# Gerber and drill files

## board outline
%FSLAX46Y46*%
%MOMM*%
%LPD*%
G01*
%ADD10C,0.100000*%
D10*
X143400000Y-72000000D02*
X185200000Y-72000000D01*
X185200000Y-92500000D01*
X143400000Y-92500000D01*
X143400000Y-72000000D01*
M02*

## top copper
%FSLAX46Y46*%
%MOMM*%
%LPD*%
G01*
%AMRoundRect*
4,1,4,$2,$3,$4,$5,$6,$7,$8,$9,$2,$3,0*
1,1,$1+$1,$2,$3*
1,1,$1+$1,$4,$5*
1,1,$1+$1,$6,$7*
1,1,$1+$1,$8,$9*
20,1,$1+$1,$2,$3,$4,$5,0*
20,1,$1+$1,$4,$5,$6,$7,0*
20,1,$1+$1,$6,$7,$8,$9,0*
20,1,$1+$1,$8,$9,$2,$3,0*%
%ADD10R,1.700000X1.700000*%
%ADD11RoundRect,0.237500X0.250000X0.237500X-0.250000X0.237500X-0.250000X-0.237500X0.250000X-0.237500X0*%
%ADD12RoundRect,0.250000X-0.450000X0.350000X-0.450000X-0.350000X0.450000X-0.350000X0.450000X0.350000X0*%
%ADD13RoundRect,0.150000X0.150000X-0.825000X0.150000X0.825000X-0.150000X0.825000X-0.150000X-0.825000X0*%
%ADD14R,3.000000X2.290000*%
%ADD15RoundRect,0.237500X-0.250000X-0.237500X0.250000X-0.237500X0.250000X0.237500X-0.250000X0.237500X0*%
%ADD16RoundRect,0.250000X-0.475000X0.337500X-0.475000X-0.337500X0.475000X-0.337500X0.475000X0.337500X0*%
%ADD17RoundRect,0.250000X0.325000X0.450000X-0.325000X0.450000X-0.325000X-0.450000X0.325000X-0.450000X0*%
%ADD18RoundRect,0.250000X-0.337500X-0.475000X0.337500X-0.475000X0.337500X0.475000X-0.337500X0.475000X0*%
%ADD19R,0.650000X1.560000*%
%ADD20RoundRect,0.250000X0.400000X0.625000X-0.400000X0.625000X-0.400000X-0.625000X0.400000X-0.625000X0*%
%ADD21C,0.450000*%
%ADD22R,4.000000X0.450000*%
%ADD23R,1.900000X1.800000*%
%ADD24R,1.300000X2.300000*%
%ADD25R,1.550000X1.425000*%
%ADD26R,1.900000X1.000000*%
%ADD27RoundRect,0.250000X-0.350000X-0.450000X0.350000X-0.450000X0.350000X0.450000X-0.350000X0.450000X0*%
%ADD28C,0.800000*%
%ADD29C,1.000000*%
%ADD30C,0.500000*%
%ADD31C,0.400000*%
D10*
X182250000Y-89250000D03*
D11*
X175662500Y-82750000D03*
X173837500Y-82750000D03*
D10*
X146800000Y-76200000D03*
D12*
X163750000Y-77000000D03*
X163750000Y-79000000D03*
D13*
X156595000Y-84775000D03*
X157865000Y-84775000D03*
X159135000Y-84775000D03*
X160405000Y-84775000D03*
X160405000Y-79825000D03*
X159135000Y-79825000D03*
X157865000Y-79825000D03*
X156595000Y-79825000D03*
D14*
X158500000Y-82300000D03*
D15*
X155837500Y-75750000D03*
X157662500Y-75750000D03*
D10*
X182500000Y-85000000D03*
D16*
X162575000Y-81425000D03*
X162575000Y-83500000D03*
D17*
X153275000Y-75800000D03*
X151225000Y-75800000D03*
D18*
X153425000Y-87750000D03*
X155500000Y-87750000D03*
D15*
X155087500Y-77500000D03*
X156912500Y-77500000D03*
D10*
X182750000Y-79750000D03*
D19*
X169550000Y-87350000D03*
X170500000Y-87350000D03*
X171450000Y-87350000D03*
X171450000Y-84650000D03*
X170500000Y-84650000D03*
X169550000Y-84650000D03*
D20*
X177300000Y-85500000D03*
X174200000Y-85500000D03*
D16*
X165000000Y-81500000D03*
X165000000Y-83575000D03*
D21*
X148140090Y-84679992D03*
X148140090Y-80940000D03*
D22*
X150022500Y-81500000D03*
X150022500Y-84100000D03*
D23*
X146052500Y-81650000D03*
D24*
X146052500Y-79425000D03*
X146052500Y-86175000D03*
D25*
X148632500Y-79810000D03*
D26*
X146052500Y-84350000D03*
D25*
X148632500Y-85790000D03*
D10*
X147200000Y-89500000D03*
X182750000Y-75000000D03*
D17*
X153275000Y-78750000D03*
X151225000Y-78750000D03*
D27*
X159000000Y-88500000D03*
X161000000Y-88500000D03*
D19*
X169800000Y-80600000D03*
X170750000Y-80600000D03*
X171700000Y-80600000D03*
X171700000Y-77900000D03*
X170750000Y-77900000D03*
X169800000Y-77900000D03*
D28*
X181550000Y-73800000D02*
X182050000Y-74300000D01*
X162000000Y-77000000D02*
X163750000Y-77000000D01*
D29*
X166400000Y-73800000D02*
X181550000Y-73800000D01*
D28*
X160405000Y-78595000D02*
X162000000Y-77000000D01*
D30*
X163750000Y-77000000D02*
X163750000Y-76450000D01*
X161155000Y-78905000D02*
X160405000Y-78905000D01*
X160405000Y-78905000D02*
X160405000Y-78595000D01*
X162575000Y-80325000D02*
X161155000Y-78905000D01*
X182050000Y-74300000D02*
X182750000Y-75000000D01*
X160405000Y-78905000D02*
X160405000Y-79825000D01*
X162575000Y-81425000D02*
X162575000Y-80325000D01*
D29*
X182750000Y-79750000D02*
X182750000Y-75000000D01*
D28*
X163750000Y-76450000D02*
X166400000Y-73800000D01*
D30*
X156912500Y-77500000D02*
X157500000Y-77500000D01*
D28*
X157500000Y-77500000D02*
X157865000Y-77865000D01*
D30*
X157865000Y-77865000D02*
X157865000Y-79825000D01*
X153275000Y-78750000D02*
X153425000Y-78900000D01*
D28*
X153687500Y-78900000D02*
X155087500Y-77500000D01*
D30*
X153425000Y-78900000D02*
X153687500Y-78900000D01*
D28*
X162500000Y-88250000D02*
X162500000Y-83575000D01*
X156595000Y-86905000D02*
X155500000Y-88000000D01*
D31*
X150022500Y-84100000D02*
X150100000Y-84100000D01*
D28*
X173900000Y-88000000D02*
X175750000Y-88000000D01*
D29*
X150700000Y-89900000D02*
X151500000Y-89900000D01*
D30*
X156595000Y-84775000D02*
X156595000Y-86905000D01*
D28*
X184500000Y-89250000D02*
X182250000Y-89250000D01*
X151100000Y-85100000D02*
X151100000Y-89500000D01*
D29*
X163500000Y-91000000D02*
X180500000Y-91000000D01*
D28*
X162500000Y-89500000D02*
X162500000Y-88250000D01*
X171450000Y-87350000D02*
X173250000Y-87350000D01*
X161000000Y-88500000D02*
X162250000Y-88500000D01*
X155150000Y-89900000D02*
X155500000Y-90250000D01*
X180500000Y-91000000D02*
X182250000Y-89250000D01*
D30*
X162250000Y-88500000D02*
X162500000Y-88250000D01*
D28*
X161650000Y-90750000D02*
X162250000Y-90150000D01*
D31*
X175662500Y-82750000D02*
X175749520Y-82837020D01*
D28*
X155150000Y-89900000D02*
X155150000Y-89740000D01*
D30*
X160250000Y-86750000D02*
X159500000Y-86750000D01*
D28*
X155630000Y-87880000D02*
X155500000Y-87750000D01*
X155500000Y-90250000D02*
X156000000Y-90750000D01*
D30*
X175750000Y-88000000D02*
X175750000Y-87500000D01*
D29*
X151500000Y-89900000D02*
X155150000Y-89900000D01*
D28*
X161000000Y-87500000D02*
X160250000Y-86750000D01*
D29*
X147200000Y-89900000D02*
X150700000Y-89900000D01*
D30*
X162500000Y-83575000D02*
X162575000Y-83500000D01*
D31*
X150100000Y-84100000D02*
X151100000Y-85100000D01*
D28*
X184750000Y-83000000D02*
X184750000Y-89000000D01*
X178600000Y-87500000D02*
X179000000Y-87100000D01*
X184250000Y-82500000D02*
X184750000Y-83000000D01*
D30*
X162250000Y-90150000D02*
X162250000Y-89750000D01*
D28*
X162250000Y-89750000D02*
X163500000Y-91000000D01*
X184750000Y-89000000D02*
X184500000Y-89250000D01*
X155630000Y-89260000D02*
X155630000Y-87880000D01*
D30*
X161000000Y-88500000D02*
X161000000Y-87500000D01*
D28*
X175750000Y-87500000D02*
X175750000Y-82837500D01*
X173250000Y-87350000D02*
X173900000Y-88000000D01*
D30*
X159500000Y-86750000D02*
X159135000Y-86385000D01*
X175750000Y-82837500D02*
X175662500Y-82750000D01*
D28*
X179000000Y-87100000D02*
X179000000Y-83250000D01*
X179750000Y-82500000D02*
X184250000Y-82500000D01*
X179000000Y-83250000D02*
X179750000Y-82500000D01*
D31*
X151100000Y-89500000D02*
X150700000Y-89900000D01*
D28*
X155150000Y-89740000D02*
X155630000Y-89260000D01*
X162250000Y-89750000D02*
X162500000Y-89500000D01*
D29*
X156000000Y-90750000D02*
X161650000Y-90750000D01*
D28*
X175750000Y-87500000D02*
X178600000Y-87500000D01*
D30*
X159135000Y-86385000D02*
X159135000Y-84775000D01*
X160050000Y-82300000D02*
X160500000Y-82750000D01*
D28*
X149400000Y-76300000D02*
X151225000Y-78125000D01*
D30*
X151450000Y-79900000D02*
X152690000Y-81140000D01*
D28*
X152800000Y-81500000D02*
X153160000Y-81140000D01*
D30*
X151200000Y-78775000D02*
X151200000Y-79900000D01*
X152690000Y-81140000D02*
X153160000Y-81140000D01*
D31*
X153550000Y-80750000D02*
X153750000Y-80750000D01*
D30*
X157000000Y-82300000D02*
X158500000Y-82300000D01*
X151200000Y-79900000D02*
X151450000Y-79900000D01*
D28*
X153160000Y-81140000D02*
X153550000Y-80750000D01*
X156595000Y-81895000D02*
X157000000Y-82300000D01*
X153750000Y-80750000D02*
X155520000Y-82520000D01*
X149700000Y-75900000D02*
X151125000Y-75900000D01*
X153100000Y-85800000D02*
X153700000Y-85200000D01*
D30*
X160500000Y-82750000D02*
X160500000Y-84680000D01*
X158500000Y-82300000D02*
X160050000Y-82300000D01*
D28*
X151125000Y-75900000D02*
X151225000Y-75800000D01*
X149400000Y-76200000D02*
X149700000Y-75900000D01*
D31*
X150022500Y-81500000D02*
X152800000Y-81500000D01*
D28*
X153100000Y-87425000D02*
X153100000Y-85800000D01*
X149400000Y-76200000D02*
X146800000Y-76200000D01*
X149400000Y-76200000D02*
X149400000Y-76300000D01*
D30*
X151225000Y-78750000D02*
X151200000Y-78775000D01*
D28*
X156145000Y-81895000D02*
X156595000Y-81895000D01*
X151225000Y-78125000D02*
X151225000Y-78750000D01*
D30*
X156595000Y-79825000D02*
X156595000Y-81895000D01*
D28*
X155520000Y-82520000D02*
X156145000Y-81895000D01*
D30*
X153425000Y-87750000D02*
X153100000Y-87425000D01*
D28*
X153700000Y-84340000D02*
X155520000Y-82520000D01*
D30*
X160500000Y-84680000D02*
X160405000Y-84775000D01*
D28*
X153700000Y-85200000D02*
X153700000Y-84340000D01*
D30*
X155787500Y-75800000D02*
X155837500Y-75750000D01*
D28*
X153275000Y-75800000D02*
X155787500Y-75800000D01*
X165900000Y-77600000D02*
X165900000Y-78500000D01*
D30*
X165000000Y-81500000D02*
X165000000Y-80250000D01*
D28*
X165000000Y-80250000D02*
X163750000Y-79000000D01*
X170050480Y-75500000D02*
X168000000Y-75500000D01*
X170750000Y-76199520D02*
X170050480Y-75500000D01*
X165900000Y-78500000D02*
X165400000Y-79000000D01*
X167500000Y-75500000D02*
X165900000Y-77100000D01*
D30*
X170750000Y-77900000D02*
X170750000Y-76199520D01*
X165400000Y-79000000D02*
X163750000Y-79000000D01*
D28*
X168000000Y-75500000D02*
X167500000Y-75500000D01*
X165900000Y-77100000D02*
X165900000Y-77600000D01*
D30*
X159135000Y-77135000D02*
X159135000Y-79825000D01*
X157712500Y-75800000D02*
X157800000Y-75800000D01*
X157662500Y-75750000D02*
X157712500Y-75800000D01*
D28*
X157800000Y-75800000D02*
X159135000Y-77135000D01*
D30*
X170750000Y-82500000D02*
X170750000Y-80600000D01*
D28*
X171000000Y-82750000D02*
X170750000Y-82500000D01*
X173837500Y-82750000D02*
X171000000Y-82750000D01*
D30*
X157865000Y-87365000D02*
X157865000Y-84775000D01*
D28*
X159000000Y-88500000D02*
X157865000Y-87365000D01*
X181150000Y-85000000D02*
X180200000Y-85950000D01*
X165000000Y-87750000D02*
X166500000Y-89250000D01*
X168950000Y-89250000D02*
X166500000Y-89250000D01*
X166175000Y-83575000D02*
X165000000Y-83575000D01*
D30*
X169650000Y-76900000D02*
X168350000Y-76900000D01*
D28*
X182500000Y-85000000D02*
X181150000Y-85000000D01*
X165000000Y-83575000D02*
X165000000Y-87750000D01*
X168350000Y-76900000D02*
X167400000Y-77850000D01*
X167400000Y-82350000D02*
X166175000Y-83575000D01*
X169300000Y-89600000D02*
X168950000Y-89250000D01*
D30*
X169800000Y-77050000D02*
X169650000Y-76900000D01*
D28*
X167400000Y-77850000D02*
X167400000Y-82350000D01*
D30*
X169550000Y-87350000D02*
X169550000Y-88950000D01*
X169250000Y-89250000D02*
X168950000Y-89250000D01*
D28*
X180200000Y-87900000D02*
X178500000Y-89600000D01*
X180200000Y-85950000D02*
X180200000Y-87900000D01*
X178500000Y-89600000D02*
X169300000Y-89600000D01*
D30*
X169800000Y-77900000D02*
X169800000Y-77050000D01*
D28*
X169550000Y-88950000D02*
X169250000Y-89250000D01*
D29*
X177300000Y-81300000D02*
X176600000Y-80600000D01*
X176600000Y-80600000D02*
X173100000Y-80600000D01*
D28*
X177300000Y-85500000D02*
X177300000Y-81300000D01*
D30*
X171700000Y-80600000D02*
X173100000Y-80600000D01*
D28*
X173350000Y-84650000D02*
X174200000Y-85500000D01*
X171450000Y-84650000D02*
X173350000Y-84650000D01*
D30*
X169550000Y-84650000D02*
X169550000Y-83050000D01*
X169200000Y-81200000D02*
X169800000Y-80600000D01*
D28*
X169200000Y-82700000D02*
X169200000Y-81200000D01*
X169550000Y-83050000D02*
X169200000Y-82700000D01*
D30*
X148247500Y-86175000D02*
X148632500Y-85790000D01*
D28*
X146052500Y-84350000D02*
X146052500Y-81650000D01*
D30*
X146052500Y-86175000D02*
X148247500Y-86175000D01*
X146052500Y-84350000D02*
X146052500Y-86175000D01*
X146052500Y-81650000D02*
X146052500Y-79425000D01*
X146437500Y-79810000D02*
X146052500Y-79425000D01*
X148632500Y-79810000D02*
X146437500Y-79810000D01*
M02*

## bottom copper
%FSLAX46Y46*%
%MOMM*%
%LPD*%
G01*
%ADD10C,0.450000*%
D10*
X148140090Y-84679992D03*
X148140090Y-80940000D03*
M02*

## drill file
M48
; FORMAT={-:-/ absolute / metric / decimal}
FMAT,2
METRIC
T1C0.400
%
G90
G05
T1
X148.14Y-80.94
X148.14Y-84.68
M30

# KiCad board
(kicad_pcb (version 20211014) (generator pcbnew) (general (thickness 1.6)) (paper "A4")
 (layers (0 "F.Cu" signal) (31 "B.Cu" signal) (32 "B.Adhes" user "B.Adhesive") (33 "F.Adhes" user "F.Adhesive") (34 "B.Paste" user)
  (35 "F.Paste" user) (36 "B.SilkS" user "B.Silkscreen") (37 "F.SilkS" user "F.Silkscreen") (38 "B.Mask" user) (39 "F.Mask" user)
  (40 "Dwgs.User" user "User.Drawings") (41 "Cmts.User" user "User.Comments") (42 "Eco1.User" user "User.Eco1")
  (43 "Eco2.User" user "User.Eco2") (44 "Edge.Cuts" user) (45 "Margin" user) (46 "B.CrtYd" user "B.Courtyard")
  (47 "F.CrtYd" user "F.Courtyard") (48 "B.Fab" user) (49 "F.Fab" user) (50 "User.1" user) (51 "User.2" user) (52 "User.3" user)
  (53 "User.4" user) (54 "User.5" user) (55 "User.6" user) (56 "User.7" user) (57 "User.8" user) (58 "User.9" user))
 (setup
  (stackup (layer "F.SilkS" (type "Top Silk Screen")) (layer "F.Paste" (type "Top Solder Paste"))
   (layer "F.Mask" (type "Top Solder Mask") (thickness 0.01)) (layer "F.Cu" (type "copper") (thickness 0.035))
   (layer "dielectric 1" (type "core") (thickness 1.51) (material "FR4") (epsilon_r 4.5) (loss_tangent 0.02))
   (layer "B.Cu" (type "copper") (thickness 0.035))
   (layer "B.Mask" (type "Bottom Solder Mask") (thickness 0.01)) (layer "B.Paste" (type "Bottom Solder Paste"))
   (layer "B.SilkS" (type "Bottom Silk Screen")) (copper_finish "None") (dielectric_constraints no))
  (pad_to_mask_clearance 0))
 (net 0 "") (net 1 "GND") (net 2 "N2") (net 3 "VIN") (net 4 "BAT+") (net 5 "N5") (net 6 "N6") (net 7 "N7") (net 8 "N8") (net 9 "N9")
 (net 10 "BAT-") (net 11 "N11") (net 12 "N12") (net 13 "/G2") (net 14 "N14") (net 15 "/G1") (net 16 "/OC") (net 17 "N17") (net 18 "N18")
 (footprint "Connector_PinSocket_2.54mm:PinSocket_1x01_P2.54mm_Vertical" (layer "F.Cu") (at 182.25 89.25)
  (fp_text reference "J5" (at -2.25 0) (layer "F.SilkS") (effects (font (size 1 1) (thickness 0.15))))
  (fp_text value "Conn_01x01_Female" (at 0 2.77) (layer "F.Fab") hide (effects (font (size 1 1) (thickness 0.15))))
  (pad "1" smd rect (at 0 0) (size 1.7 1.7) (layers "F.Cu" "F.Paste" "F.Mask") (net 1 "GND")))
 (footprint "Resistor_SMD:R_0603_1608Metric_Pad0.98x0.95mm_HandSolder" (layer "F.Cu") (at 174.75 82.75 180)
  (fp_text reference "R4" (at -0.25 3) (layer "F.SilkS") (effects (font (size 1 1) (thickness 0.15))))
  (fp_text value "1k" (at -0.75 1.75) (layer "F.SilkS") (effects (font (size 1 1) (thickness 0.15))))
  (pad "1" smd roundrect (at -0.9125 0 180) (size 0.975 0.95) (layers "F.Cu" "F.Paste" "F.Mask") (roundrect_rratio 0.25) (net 1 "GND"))
  (pad "2" smd roundrect (at 0.9125 0 180) (size 0.975 0.95) (layers "F.Cu" "F.Paste" "F.Mask") (roundrect_rratio 0.25) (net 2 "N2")))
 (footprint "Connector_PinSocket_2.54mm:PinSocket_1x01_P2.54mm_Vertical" (layer "F.Cu") (at 146.8 76.2)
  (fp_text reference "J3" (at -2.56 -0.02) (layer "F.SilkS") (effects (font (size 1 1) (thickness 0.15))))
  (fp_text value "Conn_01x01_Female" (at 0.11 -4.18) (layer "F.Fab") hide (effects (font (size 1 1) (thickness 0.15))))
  (pad "1" smd rect (at 0 0) (size 1.7 1.7) (layers "F.Cu" "F.Paste" "F.Mask") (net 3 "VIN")))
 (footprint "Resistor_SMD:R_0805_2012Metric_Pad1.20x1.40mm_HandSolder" (layer "F.Cu") (at 163.75 78 -90)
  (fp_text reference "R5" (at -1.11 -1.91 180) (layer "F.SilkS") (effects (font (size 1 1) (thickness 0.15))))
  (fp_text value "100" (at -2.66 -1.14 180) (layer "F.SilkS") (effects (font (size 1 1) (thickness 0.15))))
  (pad "1" smd roundrect (at -1 0 270) (size 1.2 1.4) (layers "F.Cu" "F.Paste" "F.Mask") (roundrect_rratio 0.2083333333) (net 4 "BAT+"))
  (pad "2" smd roundrect (at 1 0 270) (size 1.2 1.4) (layers "F.Cu" "F.Paste" "F.Mask") (roundrect_rratio 0.2083333333) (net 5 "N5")))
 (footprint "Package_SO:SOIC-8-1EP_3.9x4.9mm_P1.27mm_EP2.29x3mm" (layer "F.Cu") (at 158.5 82.3 90)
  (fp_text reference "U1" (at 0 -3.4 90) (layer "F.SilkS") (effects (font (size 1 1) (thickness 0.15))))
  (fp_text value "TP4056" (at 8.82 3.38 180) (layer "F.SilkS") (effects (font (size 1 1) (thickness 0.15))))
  (pad "" smd roundrect (at 0.57 0.75 90) (size 0.92 1.21) (layers "F.Paste") (roundrect_rratio 0.25))
  (pad "" smd roundrect (at 0.57 -0.75 90) (size 0.92 1.21) (layers "F.Paste") (roundrect_rratio 0.25))
  (pad "" smd roundrect (at -0.57 0.75 90) (size 0.92 1.21) (layers "F.Paste") (roundrect_rratio 0.25))
  (pad "" smd roundrect (at -0.57 -0.75 90) (size 0.92 1.21) (layers "F.Paste") (roundrect_rratio 0.25))
  (pad "1" smd roundrect (at -2.475 -1.905 90) (size 1.95 0.6) (layers "F.Cu" "F.Paste" "F.Mask") (roundrect_rratio 0.25) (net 1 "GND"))
  (pad "2" smd roundrect (at -2.475 -0.635 90) (size 1.95 0.6) (layers "F.Cu" "F.Paste" "F.Mask") (roundrect_rratio 0.25) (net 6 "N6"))
  (pad "3" smd roundrect (at -2.475 0.635 90) (size 1.95 0.6) (layers "F.Cu" "F.Paste" "F.Mask") (roundrect_rratio 0.25) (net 1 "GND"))
  (pad "4" smd roundrect (at -2.475 1.905 90) (size 1.95 0.6) (layers "F.Cu" "F.Paste" "F.Mask") (roundrect_rratio 0.25) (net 3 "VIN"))
  (pad "5" smd roundrect (at 2.475 1.905 90) (size 1.95 0.6) (layers "F.Cu" "F.Paste" "F.Mask") (roundrect_rratio 0.25) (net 4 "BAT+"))
  (pad "6" smd roundrect (at 2.475 0.635 90) (size 1.95 0.6) (layers "F.Cu" "F.Paste" "F.Mask") (roundrect_rratio 0.25) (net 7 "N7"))
  (pad "7" smd roundrect (at 2.475 -0.635 90) (size 1.95 0.6) (layers "F.Cu" "F.Paste" "F.Mask") (roundrect_rratio 0.25) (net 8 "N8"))
  (pad "8" smd roundrect (at 2.475 -1.905 90) (size 1.95 0.6) (layers "F.Cu" "F.Paste" "F.Mask") (roundrect_rratio 0.25) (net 3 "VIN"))
  (pad "9" smd rect (at 0 0 90) (size 2.29 3) (layers "F.Cu" "F.Mask") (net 3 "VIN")))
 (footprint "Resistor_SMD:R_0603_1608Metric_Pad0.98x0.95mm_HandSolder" (layer "F.Cu") (at 156.75 75.75)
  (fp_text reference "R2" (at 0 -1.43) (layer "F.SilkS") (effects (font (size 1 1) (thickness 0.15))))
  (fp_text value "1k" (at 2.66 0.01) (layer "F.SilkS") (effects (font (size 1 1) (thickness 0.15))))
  (pad "1" smd roundrect (at -0.9125 0) (size 0.975 0.95) (layers "F.Cu" "F.Paste" "F.Mask") (roundrect_rratio 0.25) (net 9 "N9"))
  (pad "2" smd roundrect (at 0.9125 0) (size 0.975 0.95) (layers "F.Cu" "F.Paste" "F.Mask") (roundrect_rratio 0.25) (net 7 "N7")))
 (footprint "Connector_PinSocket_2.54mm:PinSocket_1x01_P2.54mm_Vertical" (layer "F.Cu") (at 182.5 85)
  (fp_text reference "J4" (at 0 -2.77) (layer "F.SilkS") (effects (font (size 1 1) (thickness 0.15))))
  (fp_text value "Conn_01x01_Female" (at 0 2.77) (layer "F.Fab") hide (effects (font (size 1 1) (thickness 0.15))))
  (pad "1" smd rect (at 0 0) (size 1.7 1.7) (layers "F.Cu" "F.Paste" "F.Mask") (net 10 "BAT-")))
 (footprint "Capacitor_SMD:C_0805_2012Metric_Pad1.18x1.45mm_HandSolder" (layer "F.Cu") (at 162.575 82.4625 -90)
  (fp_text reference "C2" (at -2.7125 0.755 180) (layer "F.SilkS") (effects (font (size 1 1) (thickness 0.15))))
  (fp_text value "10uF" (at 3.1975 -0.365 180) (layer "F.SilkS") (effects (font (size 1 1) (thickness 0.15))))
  (pad "1" smd roundrect (at -1.0375 0 270) (size 1.175 1.45) (layers "F.Cu" "F.Paste" "F.Mask") (roundrect_rratio 0.2127659574)
   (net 4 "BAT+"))
  (pad "2" smd roundrect (at 1.0375 0 270) (size 1.175 1.45) (layers "F.Cu" "F.Paste" "F.Mask") (roundrect_rratio 0.2127659574)
   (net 1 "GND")))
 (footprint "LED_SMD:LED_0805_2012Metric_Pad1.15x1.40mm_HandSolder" (layer "F.Cu") (at 152.25 75.8 180)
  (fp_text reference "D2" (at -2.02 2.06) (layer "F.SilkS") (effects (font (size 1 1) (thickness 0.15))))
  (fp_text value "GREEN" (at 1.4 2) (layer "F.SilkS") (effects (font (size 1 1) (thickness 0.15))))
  (pad "1" smd roundrect (at -1.025 0 180) (size 1.15 1.4) (layers "F.Cu" "F.Paste" "F.Mask") (roundrect_rratio 0.2173913043) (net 9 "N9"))
  (pad "2" smd roundrect (at 1.025 0 180) (size 1.15 1.4) (layers "F.Cu" "F.Paste" "F.Mask") (roundrect_rratio 0.2173913043) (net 3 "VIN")))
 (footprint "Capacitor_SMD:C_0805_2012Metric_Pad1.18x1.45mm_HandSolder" (layer "F.Cu") (at 154.4625 87.75)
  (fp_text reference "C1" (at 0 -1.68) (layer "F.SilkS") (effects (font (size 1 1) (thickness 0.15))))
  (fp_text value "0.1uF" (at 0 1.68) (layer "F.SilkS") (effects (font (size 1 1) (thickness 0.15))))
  (pad "1" smd roundrect (at -1.0375 0) (size 1.175 1.45) (layers "F.Cu" "F.Paste" "F.Mask") (roundrect_rratio 0.2127659574) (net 3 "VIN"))
  (pad "2" smd roundrect (at 1.0375 0) (size 1.175 1.45) (layers "F.Cu" "F.Paste" "F.Mask") (roundrect_rratio 0.2127659574) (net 1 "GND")))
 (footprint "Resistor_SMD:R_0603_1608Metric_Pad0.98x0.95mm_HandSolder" (layer "F.Cu") (at 156 77.5)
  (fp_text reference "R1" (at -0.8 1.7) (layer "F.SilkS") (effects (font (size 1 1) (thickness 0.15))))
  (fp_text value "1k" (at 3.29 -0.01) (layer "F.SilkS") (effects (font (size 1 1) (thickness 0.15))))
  (pad "1" smd roundrect (at -0.9125 0) (size 0.975 0.95) (layers "F.Cu" "F.Paste" "F.Mask") (roundrect_rratio 0.25) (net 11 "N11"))
  (pad "2" smd roundrect (at 0.9125 0) (size 0.975 0.95) (layers "F.Cu" "F.Paste" "F.Mask") (roundrect_rratio 0.25) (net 8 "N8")))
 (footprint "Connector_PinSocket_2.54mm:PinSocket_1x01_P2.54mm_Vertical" (layer "F.Cu") (at 182.75 79.75)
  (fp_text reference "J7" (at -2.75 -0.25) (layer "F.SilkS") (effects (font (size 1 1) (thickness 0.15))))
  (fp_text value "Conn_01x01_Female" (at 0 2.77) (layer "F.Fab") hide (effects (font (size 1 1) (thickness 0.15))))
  (pad "1" smd rect (at 0 0) (size 1.7 1.7) (layers "F.Cu" "F.Paste" "F.Mask") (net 4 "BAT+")))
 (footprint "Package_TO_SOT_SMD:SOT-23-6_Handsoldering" (layer "F.Cu") (at 170.5 86 90)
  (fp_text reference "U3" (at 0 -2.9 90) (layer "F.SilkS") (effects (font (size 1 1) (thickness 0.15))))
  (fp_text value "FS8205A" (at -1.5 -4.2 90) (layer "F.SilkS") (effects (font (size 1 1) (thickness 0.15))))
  (pad "1" smd rect (at -1.35 -0.95 90) (size 1.56 0.65) (layers "F.Cu" "F.Paste" "F.Mask") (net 10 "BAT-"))
  (pad "2" smd rect (at -1.35 0 90) (size 1.56 0.65) (layers "F.Cu" "F.Paste" "F.Mask") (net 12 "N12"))
  (pad "3" smd rect (at -1.35 0.95 90) (size 1.56 0.65) (layers "F.Cu" "F.Paste" "F.Mask") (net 1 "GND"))
  (pad "4" smd rect (at 1.35 0.95 90) (size 1.56 0.65) (layers "F.Cu" "F.Paste" "F.Mask") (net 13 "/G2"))
  (pad "5" smd rect (at 1.35 0 90) (size 1.56 0.65) (layers "F.Cu" "F.Paste" "F.Mask") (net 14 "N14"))
  (pad "6" smd rect (at 1.35 -0.95 90) (size 1.56 0.65) (layers "F.Cu" "F.Paste" "F.Mask") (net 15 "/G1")))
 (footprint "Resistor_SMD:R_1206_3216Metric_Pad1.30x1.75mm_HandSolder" (layer "F.Cu") (at 175.75 85.5 180)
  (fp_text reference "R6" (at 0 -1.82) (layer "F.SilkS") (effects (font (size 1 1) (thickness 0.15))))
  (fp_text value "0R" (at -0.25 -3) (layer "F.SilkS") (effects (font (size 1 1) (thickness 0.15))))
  (pad "1" smd roundrect (at -1.55 0 180) (size 1.3 1.75) (layers "F.Cu" "F.Paste" "F.Mask") (roundrect_rratio 0.1923076923) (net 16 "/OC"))
  (pad "2" smd roundrect (at 1.55 0 180) (size 1.3 1.75) (layers "F.Cu" "F.Paste" "F.Mask") (roundrect_rratio 0.1923076923) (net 13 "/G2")))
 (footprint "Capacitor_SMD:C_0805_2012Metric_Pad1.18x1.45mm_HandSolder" (layer "F.Cu") (at 165 82.5375 -90)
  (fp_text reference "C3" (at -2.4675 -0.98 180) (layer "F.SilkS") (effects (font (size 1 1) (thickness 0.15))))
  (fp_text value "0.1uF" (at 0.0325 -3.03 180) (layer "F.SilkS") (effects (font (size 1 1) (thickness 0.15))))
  (pad "1" smd roundrect (at -1.0375 0 270) (size 1.175 1.45) (layers "F.Cu" "F.Paste" "F.Mask") (roundrect_rratio 0.2127659574)
   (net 5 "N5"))
  (pad "2" smd roundrect (at 1.0375 0 270) (size 1.175 1.45) (layers "F.Cu" "F.Paste" "F.Mask") (roundrect_rratio 0.2127659574)
   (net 10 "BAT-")))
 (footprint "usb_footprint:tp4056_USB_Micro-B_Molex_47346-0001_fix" (layer "F.Cu") (at 147.2525 82.8 -90)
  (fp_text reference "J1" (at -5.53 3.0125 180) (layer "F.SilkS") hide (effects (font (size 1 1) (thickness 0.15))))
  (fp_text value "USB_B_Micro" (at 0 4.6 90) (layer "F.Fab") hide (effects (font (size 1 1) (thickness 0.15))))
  (pad "" np_thru_hole circle (at 1.879992 -0.88759 270) (size 0.45 0.45) (drill 0.4) (layers F&B.Cu *.Mask) (clearance 0.02))
  (pad "" np_thru_hole circle (at -1.86 -0.88759 270) (size 0.45 0.45) (drill 0.4) (layers F&B.Cu *.Mask) (clearance 0.02))
  (pad "1" smd rect (at -1.3 -2.77 270) (size 0.45 4) (layers "F.Cu" "F.Paste" "F.Mask") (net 3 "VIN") (clearance 0.02))
  (pad "5" smd rect (at 1.3 -2.77 270) (size 0.45 4) (layers "F.Cu" "F.Paste" "F.Mask") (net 1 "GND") (clearance 0.02))
  (pad "6" smd rect (at -1.15 1.2 270) (size 1.8 1.9) (layers "F.Cu" "F.Paste" "F.Mask") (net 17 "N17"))
  (pad "6" smd rect (at -3.375 1.2 270) (size 2.3 1.3) (layers "F.Cu" "F.Paste" "F.Mask") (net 17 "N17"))
  (pad "6" smd rect (at 3.375 1.2 270) (size 2.3 1.3) (layers "F.Cu" "F.Paste" "F.Mask") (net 17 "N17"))
  (pad "6" smd rect (at -2.99 -1.38 270) (size 1.425 1.55) (layers "F.Cu" "F.Paste" "F.Mask") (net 17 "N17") (clearance 0.02))
  (pad "6" smd rect (at 1.55 1.2 270) (size 1 1.9) (layers "F.Cu" "F.Paste" "F.Mask") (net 17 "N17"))
  (pad "6" smd rect (at 2.99 -1.38 270) (size 1.425 1.55) (layers "F.Cu" "F.Paste" "F.Mask") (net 17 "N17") (clearance 0.02)))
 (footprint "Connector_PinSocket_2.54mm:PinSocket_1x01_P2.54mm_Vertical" (layer "F.Cu") (at 147.2 89.5)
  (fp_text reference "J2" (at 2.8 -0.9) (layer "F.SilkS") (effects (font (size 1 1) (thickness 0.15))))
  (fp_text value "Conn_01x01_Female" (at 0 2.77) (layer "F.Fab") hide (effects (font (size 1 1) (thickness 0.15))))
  (pad "1" smd rect (at 0 0) (size 1.7 1.7) (layers "F.Cu" "F.Paste" "F.Mask") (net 1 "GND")))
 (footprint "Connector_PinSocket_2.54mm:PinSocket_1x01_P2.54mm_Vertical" (layer "F.Cu") (at 182.75 75)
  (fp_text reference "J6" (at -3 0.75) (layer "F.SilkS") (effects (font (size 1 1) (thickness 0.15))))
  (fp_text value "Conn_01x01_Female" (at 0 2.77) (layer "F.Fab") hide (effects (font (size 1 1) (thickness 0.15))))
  (pad "1" smd rect (at 0 0) (size 1.7 1.7) (layers "F.Cu" "F.Paste" "F.Mask") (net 4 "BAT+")))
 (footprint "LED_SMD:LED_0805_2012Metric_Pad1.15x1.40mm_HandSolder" (layer "F.Cu") (at 152.25 78.75 180)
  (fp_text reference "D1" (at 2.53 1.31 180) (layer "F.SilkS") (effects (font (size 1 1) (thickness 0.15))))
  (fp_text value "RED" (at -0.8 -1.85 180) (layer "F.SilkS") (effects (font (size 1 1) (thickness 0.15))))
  (pad "1" smd roundrect (at -1.025 0 180) (size 1.15 1.4) (layers "F.Cu" "F.Paste" "F.Mask") (roundrect_rratio 0.2173913043) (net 11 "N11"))
  (pad "2" smd roundrect (at 1.025 0 180) (size 1.15 1.4) (layers "F.Cu" "F.Paste" "F.Mask") (roundrect_rratio 0.2173913043) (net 3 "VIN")))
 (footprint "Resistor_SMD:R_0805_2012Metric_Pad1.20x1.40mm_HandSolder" (layer "F.Cu") (at 160 88.5)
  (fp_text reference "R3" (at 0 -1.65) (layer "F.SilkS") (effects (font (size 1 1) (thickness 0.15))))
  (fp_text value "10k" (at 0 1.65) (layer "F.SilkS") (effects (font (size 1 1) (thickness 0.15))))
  (pad "1" smd roundrect (at -1 0) (size 1.2 1.4) (layers "F.Cu" "F.Paste" "F.Mask") (roundrect_rratio 0.2083333333) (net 6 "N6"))
  (pad "2" smd roundrect (at 1 0) (size 1.2 1.4) (layers "F.Cu" "F.Paste" "F.Mask") (roundrect_rratio 0.2083333333) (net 1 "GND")))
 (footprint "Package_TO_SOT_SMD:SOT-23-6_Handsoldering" (layer "F.Cu") (at 170.75 79.25 90)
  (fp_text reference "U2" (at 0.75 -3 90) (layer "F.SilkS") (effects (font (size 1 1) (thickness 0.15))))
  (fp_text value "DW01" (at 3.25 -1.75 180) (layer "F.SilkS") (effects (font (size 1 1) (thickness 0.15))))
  (pad "1" smd rect (at -1.35 -0.95 90) (size 1.56 0.65) (layers "F.Cu" "F.Paste" "F.Mask") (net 15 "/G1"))
  (pad "2" smd rect (at -1.35 0 90) (size 1.56 0.65) (layers "F.Cu" "F.Paste" "F.Mask") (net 2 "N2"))
  (pad "3" smd rect (at -1.35 0.95 90) (size 1.56 0.65) (layers "F.Cu" "F.Paste" "F.Mask") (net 16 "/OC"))
  (pad "4" smd rect (at 1.35 0.95 90) (size 1.56 0.65) (layers "F.Cu" "F.Paste" "F.Mask") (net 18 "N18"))
  (pad "5" smd rect (at 1.35 0 90) (size 1.56 0.65) (layers "F.Cu" "F.Paste" "F.Mask") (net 5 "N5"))
  (pad "6" smd rect (at 1.35 -0.95 90) (size 1.56 0.65) (layers "F.Cu" "F.Paste" "F.Mask") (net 10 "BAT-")))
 (gr_rect (start 143.4 72) (end 185.2 92.5) (layer "Edge.Cuts") (width 0.1) (fill none))
 (segment (start 181.55 73.8) (end 182.05 74.3) (width 0.8) (layer "F.Cu") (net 4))
 (segment (start 162 77) (end 163.75 77) (width 0.8) (layer "F.Cu") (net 4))
 (segment (start 166.4 73.8) (end 181.55 73.8) (width 1) (layer "F.Cu") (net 4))
 (segment (start 160.405 78.595) (end 162 77) (width 0.8) (layer "F.Cu") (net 4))
 (segment (start 163.75 77) (end 163.75 76.45) (width 0.5) (layer "F.Cu") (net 4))
 (segment (start 161.155 78.905) (end 160.405 78.905) (width 0.5) (layer "F.Cu") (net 4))
 (segment (start 160.405 78.905) (end 160.405 78.595) (width 0.5) (layer "F.Cu") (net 4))
 (segment (start 162.575 80.325) (end 161.155 78.905) (width 0.5) (layer "F.Cu") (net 4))
 (segment (start 182.05 74.3) (end 182.75 75) (width 0.5) (layer "F.Cu") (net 4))
 (segment (start 160.405 78.905) (end 160.405 79.825) (width 0.5) (layer "F.Cu") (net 4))
 (segment (start 162.575 81.425) (end 162.575 80.325) (width 0.5) (layer "F.Cu") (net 4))
 (segment (start 182.75 79.75) (end 182.75 75) (width 1) (layer "F.Cu") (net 4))
 (segment (start 163.75 76.45) (end 166.4 73.8) (width 0.8) (layer "F.Cu") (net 4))
 (segment (start 156.9125 77.5) (end 157.5 77.5) (width 0.5) (layer "F.Cu") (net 8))
 (segment (start 157.5 77.5) (end 157.865 77.865) (width 0.8) (layer "F.Cu") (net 8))
 (segment (start 157.865 77.865) (end 157.865 79.825) (width 0.5) (layer "F.Cu") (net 8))
 (segment (start 153.275 78.75) (end 153.425 78.9) (width 0.5) (layer "F.Cu") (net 11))
 (segment (start 153.6875 78.9) (end 155.0875 77.5) (width 0.8) (layer "F.Cu") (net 11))
 (segment (start 153.425 78.9) (end 153.6875 78.9) (width 0.5) (layer "F.Cu") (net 11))
 (segment (start 162.5 88.25) (end 162.5 83.575) (width 0.8) (layer "F.Cu") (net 1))
 (segment (start 156.595 86.905) (end 155.5 88) (width 0.8) (layer "F.Cu") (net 1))
 (segment (start 150.0225 84.1) (end 150.1 84.1) (width 0.4) (layer "F.Cu") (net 1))
 (segment (start 173.9 88) (end 175.75 88) (width 0.8) (layer "F.Cu") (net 1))
 (segment (start 150.7 89.9) (end 151.5 89.9) (width 1) (layer "F.Cu") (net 1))
 (segment (start 156.595 84.775) (end 156.595 86.905) (width 0.5) (layer "F.Cu") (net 1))
 (segment (start 184.5 89.25) (end 182.25 89.25) (width 0.8) (layer "F.Cu") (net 1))
 (segment (start 151.1 85.1) (end 151.1 89.5) (width 0.8) (layer "F.Cu") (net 1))
 (segment (start 163.5 91) (end 180.5 91) (width 1) (layer "F.Cu") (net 1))
 (segment (start 162.5 89.5) (end 162.5 88.25) (width 0.8) (layer "F.Cu") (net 1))
 (segment (start 171.45 87.35) (end 173.25 87.35) (width 0.8) (layer "F.Cu") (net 1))
 (segment (start 161 88.5) (end 162.25 88.5) (width 0.8) (layer "F.Cu") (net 1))
 (segment (start 155.15 89.9) (end 155.5 90.25) (width 0.8) (layer "F.Cu") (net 1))
 (segment (start 180.5 91) (end 182.25 89.25) (width 0.8) (layer "F.Cu") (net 1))
 (segment (start 162.25 88.5) (end 162.5 88.25) (width 0.5) (layer "F.Cu") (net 1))
 (segment (start 161.65 90.75) (end 162.25 90.15) (width 0.8) (layer "F.Cu") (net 1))
 (segment (start 175.6625 82.75) (end 175.74952 82.83702) (width 0.4) (layer "F.Cu") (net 1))
 (segment (start 155.15 89.9) (end 155.15 89.74) (width 0.8) (layer "F.Cu") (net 1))
 (segment (start 160.25 86.75) (end 159.5 86.75) (width 0.5) (layer "F.Cu") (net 1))
 (segment (start 155.63 87.88) (end 155.5 87.75) (width 0.8) (layer "F.Cu") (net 1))
 (segment (start 155.5 90.25) (end 156 90.75) (width 0.8) (layer "F.Cu") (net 1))
 (segment (start 175.75 88) (end 175.75 87.5) (width 0.5) (layer "F.Cu") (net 1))
 (segment (start 151.5 89.9) (end 155.15 89.9) (width 1) (layer "F.Cu") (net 1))
 (segment (start 161 87.5) (end 160.25 86.75) (width 0.8) (layer "F.Cu") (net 1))
 (segment (start 147.2 89.9) (end 150.7 89.9) (width 1) (layer "F.Cu") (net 1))
 (segment (start 162.5 83.575) (end 162.575 83.5) (width 0.5) (layer "F.Cu") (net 1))
 (segment (start 150.1 84.1) (end 151.1 85.1) (width 0.4) (layer "F.Cu") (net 1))
 (segment (start 184.75 83) (end 184.75 89) (width 0.8) (layer "F.Cu") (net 1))
 (segment (start 178.6 87.5) (end 179 87.1) (width 0.8) (layer "F.Cu") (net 1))
 (segment (start 184.25 82.5) (end 184.75 83) (width 0.8) (layer "F.Cu") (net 1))
 (segment (start 162.25 90.15) (end 162.25 89.75) (width 0.5) (layer "F.Cu") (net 1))
 (segment (start 162.25 89.75) (end 163.5 91) (width 0.8) (layer "F.Cu") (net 1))
 (segment (start 184.75 89) (end 184.5 89.25) (width 0.8) (layer "F.Cu") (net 1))
 (segment (start 155.63 89.26) (end 155.63 87.88) (width 0.8) (layer "F.Cu") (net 1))
 (segment (start 161 88.5) (end 161 87.5) (width 0.5) (layer "F.Cu") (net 1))
 (segment (start 175.75 87.5) (end 175.75 82.8375) (width 0.8) (layer "F.Cu") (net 1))
 (segment (start 173.25 87.35) (end 173.9 88) (width 0.8) (layer "F.Cu") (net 1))
 (segment (start 159.5 86.75) (end 159.135 86.385) (width 0.5) (layer "F.Cu") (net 1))
 (segment (start 175.75 82.8375) (end 175.6625 82.75) (width 0.5) (layer "F.Cu") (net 1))
 (segment (start 179 87.1) (end 179 83.25) (width 0.8) (layer "F.Cu") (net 1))
 (segment (start 179.75 82.5) (end 184.25 82.5) (width 0.8) (layer "F.Cu") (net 1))
 (segment (start 179 83.25) (end 179.75 82.5) (width 0.8) (layer "F.Cu") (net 1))
 (segment (start 151.1 89.5) (end 150.7 89.9) (width 0.4) (layer "F.Cu") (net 1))
 (segment (start 155.15 89.74) (end 155.63 89.26) (width 0.8) (layer "F.Cu") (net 1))
 (segment (start 162.25 89.75) (end 162.5 89.5) (width 0.8) (layer "F.Cu") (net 1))
 (segment (start 156 90.75) (end 161.65 90.75) (width 1) (layer "F.Cu") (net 1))
 (segment (start 175.75 87.5) (end 178.6 87.5) (width 0.8) (layer "F.Cu") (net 1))
 (segment (start 159.135 86.385) (end 159.135 84.775) (width 0.5) (layer "F.Cu") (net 1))
 (segment (start 160.05 82.3) (end 160.5 82.75) (width 0.5) (layer "F.Cu") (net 3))
 (segment (start 149.4 76.3) (end 151.225 78.125) (width 0.8) (layer "F.Cu") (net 3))
 (segment (start 151.45 79.9) (end 152.69 81.14) (width 0.5) (layer "F.Cu") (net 3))
 (segment (start 152.8 81.5) (end 153.16 81.14) (width 0.8) (layer "F.Cu") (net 3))
 (segment (start 151.2 78.775) (end 151.2 79.9) (width 0.5) (layer "F.Cu") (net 3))
 (segment (start 152.69 81.14) (end 153.16 81.14) (width 0.5) (layer "F.Cu") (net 3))
 (segment (start 153.55 80.75) (end 153.75 80.75) (width 0.4) (layer "F.Cu") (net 3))
 (segment (start 157 82.3) (end 158.5 82.3) (width 0.5) (layer "F.Cu") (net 3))
 (segment (start 151.2 79.9) (end 151.45 79.9) (width 0.5) (layer "F.Cu") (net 3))
 (segment (start 153.16 81.14) (end 153.55 80.75) (width 0.8) (layer "F.Cu") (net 3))
 (segment (start 156.595 81.895) (end 157 82.3) (width 0.8) (layer "F.Cu") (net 3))
 (segment (start 153.75 80.75) (end 155.52 82.52) (width 0.8) (layer "F.Cu") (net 3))
 (segment (start 149.7 75.9) (end 151.125 75.9) (width 0.8) (layer "F.Cu") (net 3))
 (segment (start 153.1 85.8) (end 153.7 85.2) (width 0.8) (layer "F.Cu") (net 3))
 (segment (start 160.5 82.75) (end 160.5 84.68) (width 0.5) (layer "F.Cu") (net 3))
 (segment (start 158.5 82.3) (end 160.05 82.3) (width 0.5) (layer "F.Cu") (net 3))
 (segment (start 151.125 75.9) (end 151.225 75.8) (width 0.8) (layer "F.Cu") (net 3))
 (segment (start 149.4 76.2) (end 149.7 75.9) (width 0.8) (layer "F.Cu") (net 3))
 (segment (start 150.0225 81.5) (end 152.8 81.5) (width 0.4) (layer "F.Cu") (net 3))
 (segment (start 153.1 87.425) (end 153.1 85.8) (width 0.8) (layer "F.Cu") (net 3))
 (segment (start 149.4 76.2) (end 146.8 76.2) (width 0.8) (layer "F.Cu") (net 3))
 (segment (start 149.4 76.2) (end 149.4 76.3) (width 0.8) (layer "F.Cu") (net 3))
 (segment (start 151.225 78.75) (end 151.2 78.775) (width 0.5) (layer "F.Cu") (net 3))
 (segment (start 156.145 81.895) (end 156.595 81.895) (width 0.8) (layer "F.Cu") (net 3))
 (segment (start 151.225 78.125) (end 151.225 78.75) (width 0.8) (layer "F.Cu") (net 3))
 (segment (start 156.595 79.825) (end 156.595 81.895) (width 0.5) (layer "F.Cu") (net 3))
 (segment (start 155.52 82.52) (end 156.145 81.895) (width 0.8) (layer "F.Cu") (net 3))
 (segment (start 153.425 87.75) (end 153.1 87.425) (width 0.5) (layer "F.Cu") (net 3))
 (segment (start 153.7 84.34) (end 155.52 82.52) (width 0.8) (layer "F.Cu") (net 3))
 (segment (start 160.5 84.68) (end 160.405 84.775) (width 0.5) (layer "F.Cu") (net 3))
 (segment (start 153.7 85.2) (end 153.7 84.34) (width 0.8) (layer "F.Cu") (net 3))
 (segment (start 155.7875 75.8) (end 155.8375 75.75) (width 0.5) (layer "F.Cu") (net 9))
 (segment (start 153.275 75.8) (end 155.7875 75.8) (width 0.8) (layer "F.Cu") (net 9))
 (segment (start 165.9 77.6) (end 165.9 78.5) (width 0.8) (layer "F.Cu") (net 5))
 (segment (start 165 81.5) (end 165 80.25) (width 0.5) (layer "F.Cu") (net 5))
 (segment (start 165 80.25) (end 163.75 79) (width 0.8) (layer "F.Cu") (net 5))
 (segment (start 170.05048 75.5) (end 168 75.5) (width 0.8) (layer "F.Cu") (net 5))
 (segment (start 170.75 76.19952) (end 170.05048 75.5) (width 0.8) (layer "F.Cu") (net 5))
 (segment (start 165.9 78.5) (end 165.4 79) (width 0.8) (layer "F.Cu") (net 5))
 (segment (start 167.5 75.5) (end 165.9 77.1) (width 0.8) (layer "F.Cu") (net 5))
 (segment (start 170.75 77.9) (end 170.75 76.19952) (width 0.5) (layer "F.Cu") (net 5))
 (segment (start 165.4 79) (end 163.75 79) (width 0.5) (layer "F.Cu") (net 5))
 (segment (start 168 75.5) (end 167.5 75.5) (width 0.8) (layer "F.Cu") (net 5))
 (segment (start 165.9 77.1) (end 165.9 77.6) (width 0.8) (layer "F.Cu") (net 5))
 (segment (start 159.135 77.135) (end 159.135 79.825) (width 0.5) (layer "F.Cu") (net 7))
 (segment (start 157.7125 75.8) (end 157.8 75.8) (width 0.5) (layer "F.Cu") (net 7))
 (segment (start 157.6625 75.75) (end 157.7125 75.8) (width 0.5) (layer "F.Cu") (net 7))
 (segment (start 157.8 75.8) (end 159.135 77.135) (width 0.8) (layer "F.Cu") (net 7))
 (segment (start 170.75 82.5) (end 170.75 80.6) (width 0.5) (layer "F.Cu") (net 2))
 (segment (start 171 82.75) (end 170.75 82.5) (width 0.8) (layer "F.Cu") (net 2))
 (segment (start 173.8375 82.75) (end 171 82.75) (width 0.8) (layer "F.Cu") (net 2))
 (segment (start 157.865 87.365) (end 157.865 84.775) (width 0.5) (layer "F.Cu") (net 6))
 (segment (start 159 88.5) (end 157.865 87.365) (width 0.8) (layer "F.Cu") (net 6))
 (segment (start 181.15 85) (end 180.2 85.95) (width 0.8) (layer "F.Cu") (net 10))
 (segment (start 165 87.75) (end 166.5 89.25) (width 0.8) (layer "F.Cu") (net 10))
 (segment (start 168.95 89.25) (end 166.5 89.25) (width 0.8) (layer "F.Cu") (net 10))
 (segment (start 166.175 83.575) (end 165 83.575) (width 0.8) (layer "F.Cu") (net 10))
 (segment (start 169.65 76.9) (end 168.35 76.9) (width 0.5) (layer "F.Cu") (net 10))
 (segment (start 182.5 85) (end 181.15 85) (width 0.8) (layer "F.Cu") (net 10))
 (segment (start 165 83.575) (end 165 87.75) (width 0.8) (layer "F.Cu") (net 10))
 (segment (start 168.35 76.9) (end 167.4 77.85) (width 0.8) (layer "F.Cu") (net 10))
 (segment (start 167.4 82.35) (end 166.175 83.575) (width 0.8) (layer "F.Cu") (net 10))
 (segment (start 169.3 89.6) (end 168.95 89.25) (width 0.8) (layer "F.Cu") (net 10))
 (segment (start 169.8 77.05) (end 169.65 76.9) (width 0.5) (layer "F.Cu") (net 10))
 (segment (start 167.4 77.85) (end 167.4 82.35) (width 0.8) (layer "F.Cu") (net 10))
 (segment (start 169.55 87.35) (end 169.55 88.95) (width 0.5) (layer "F.Cu") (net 10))
 (segment (start 169.25 89.25) (end 168.95 89.25) (width 0.5) (layer "F.Cu") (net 10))
 (segment (start 180.2 87.9) (end 178.5 89.6) (width 0.8) (layer "F.Cu") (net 10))
 (segment (start 180.2 85.95) (end 180.2 87.9) (width 0.8) (layer "F.Cu") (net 10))
 (segment (start 178.5 89.6) (end 169.3 89.6) (width 0.8) (layer "F.Cu") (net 10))
 (segment (start 169.8 77.9) (end 169.8 77.05) (width 0.5) (layer "F.Cu") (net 10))
 (segment (start 169.55 88.95) (end 169.25 89.25) (width 0.8) (layer "F.Cu") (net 10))
 (segment (start 177.3 81.3) (end 176.6 80.6) (width 1) (layer "F.Cu") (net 16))
 (segment (start 176.6 80.6) (end 173.1 80.6) (width 1) (layer "F.Cu") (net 16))
 (segment (start 177.3 85.5) (end 177.3 81.3) (width 0.8) (layer "F.Cu") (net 16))
 (segment (start 171.7 80.6) (end 173.1 80.6) (width 0.5) (layer "F.Cu") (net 16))
 (segment (start 173.35 84.65) (end 174.2 85.5) (width 0.8) (layer "F.Cu") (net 13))
 (segment (start 171.45 84.65) (end 173.35 84.65) (width 0.8) (layer "F.Cu") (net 13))
 (segment (start 169.55 84.65) (end 169.55 83.05) (width 0.5) (layer "F.Cu") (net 15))
 (segment (start 169.2 81.2) (end 169.8 80.6) (width 0.5) (layer "F.Cu") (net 15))
 (segment (start 169.2 82.7) (end 169.2 81.2) (width 0.8) (layer "F.Cu") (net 15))
 (segment (start 169.55 83.05) (end 169.2 82.7) (width 0.8) (layer "F.Cu") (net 15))
 (segment (start 148.2475 86.175) (end 148.6325 85.79) (width 0.5) (layer "F.Cu") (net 17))
 (segment (start 146.0525 84.35) (end 146.0525 81.65) (width 0.8) (layer "F.Cu") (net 17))
 (segment (start 146.0525 86.175) (end 148.2475 86.175) (width 0.5) (layer "F.Cu") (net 17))
 (segment (start 146.0525 84.35) (end 146.0525 86.175) (width 0.5) (layer "F.Cu") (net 17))
 (segment (start 146.0525 81.65) (end 146.0525 79.425) (width 0.5) (layer "F.Cu") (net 17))
 (segment (start 146.4375 79.81) (end 146.0525 79.425) (width 0.5) (layer "F.Cu") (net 17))
 (segment (start 148.6325 79.81) (end 146.4375 79.81) (width 0.5) (layer "F.Cu") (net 17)))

